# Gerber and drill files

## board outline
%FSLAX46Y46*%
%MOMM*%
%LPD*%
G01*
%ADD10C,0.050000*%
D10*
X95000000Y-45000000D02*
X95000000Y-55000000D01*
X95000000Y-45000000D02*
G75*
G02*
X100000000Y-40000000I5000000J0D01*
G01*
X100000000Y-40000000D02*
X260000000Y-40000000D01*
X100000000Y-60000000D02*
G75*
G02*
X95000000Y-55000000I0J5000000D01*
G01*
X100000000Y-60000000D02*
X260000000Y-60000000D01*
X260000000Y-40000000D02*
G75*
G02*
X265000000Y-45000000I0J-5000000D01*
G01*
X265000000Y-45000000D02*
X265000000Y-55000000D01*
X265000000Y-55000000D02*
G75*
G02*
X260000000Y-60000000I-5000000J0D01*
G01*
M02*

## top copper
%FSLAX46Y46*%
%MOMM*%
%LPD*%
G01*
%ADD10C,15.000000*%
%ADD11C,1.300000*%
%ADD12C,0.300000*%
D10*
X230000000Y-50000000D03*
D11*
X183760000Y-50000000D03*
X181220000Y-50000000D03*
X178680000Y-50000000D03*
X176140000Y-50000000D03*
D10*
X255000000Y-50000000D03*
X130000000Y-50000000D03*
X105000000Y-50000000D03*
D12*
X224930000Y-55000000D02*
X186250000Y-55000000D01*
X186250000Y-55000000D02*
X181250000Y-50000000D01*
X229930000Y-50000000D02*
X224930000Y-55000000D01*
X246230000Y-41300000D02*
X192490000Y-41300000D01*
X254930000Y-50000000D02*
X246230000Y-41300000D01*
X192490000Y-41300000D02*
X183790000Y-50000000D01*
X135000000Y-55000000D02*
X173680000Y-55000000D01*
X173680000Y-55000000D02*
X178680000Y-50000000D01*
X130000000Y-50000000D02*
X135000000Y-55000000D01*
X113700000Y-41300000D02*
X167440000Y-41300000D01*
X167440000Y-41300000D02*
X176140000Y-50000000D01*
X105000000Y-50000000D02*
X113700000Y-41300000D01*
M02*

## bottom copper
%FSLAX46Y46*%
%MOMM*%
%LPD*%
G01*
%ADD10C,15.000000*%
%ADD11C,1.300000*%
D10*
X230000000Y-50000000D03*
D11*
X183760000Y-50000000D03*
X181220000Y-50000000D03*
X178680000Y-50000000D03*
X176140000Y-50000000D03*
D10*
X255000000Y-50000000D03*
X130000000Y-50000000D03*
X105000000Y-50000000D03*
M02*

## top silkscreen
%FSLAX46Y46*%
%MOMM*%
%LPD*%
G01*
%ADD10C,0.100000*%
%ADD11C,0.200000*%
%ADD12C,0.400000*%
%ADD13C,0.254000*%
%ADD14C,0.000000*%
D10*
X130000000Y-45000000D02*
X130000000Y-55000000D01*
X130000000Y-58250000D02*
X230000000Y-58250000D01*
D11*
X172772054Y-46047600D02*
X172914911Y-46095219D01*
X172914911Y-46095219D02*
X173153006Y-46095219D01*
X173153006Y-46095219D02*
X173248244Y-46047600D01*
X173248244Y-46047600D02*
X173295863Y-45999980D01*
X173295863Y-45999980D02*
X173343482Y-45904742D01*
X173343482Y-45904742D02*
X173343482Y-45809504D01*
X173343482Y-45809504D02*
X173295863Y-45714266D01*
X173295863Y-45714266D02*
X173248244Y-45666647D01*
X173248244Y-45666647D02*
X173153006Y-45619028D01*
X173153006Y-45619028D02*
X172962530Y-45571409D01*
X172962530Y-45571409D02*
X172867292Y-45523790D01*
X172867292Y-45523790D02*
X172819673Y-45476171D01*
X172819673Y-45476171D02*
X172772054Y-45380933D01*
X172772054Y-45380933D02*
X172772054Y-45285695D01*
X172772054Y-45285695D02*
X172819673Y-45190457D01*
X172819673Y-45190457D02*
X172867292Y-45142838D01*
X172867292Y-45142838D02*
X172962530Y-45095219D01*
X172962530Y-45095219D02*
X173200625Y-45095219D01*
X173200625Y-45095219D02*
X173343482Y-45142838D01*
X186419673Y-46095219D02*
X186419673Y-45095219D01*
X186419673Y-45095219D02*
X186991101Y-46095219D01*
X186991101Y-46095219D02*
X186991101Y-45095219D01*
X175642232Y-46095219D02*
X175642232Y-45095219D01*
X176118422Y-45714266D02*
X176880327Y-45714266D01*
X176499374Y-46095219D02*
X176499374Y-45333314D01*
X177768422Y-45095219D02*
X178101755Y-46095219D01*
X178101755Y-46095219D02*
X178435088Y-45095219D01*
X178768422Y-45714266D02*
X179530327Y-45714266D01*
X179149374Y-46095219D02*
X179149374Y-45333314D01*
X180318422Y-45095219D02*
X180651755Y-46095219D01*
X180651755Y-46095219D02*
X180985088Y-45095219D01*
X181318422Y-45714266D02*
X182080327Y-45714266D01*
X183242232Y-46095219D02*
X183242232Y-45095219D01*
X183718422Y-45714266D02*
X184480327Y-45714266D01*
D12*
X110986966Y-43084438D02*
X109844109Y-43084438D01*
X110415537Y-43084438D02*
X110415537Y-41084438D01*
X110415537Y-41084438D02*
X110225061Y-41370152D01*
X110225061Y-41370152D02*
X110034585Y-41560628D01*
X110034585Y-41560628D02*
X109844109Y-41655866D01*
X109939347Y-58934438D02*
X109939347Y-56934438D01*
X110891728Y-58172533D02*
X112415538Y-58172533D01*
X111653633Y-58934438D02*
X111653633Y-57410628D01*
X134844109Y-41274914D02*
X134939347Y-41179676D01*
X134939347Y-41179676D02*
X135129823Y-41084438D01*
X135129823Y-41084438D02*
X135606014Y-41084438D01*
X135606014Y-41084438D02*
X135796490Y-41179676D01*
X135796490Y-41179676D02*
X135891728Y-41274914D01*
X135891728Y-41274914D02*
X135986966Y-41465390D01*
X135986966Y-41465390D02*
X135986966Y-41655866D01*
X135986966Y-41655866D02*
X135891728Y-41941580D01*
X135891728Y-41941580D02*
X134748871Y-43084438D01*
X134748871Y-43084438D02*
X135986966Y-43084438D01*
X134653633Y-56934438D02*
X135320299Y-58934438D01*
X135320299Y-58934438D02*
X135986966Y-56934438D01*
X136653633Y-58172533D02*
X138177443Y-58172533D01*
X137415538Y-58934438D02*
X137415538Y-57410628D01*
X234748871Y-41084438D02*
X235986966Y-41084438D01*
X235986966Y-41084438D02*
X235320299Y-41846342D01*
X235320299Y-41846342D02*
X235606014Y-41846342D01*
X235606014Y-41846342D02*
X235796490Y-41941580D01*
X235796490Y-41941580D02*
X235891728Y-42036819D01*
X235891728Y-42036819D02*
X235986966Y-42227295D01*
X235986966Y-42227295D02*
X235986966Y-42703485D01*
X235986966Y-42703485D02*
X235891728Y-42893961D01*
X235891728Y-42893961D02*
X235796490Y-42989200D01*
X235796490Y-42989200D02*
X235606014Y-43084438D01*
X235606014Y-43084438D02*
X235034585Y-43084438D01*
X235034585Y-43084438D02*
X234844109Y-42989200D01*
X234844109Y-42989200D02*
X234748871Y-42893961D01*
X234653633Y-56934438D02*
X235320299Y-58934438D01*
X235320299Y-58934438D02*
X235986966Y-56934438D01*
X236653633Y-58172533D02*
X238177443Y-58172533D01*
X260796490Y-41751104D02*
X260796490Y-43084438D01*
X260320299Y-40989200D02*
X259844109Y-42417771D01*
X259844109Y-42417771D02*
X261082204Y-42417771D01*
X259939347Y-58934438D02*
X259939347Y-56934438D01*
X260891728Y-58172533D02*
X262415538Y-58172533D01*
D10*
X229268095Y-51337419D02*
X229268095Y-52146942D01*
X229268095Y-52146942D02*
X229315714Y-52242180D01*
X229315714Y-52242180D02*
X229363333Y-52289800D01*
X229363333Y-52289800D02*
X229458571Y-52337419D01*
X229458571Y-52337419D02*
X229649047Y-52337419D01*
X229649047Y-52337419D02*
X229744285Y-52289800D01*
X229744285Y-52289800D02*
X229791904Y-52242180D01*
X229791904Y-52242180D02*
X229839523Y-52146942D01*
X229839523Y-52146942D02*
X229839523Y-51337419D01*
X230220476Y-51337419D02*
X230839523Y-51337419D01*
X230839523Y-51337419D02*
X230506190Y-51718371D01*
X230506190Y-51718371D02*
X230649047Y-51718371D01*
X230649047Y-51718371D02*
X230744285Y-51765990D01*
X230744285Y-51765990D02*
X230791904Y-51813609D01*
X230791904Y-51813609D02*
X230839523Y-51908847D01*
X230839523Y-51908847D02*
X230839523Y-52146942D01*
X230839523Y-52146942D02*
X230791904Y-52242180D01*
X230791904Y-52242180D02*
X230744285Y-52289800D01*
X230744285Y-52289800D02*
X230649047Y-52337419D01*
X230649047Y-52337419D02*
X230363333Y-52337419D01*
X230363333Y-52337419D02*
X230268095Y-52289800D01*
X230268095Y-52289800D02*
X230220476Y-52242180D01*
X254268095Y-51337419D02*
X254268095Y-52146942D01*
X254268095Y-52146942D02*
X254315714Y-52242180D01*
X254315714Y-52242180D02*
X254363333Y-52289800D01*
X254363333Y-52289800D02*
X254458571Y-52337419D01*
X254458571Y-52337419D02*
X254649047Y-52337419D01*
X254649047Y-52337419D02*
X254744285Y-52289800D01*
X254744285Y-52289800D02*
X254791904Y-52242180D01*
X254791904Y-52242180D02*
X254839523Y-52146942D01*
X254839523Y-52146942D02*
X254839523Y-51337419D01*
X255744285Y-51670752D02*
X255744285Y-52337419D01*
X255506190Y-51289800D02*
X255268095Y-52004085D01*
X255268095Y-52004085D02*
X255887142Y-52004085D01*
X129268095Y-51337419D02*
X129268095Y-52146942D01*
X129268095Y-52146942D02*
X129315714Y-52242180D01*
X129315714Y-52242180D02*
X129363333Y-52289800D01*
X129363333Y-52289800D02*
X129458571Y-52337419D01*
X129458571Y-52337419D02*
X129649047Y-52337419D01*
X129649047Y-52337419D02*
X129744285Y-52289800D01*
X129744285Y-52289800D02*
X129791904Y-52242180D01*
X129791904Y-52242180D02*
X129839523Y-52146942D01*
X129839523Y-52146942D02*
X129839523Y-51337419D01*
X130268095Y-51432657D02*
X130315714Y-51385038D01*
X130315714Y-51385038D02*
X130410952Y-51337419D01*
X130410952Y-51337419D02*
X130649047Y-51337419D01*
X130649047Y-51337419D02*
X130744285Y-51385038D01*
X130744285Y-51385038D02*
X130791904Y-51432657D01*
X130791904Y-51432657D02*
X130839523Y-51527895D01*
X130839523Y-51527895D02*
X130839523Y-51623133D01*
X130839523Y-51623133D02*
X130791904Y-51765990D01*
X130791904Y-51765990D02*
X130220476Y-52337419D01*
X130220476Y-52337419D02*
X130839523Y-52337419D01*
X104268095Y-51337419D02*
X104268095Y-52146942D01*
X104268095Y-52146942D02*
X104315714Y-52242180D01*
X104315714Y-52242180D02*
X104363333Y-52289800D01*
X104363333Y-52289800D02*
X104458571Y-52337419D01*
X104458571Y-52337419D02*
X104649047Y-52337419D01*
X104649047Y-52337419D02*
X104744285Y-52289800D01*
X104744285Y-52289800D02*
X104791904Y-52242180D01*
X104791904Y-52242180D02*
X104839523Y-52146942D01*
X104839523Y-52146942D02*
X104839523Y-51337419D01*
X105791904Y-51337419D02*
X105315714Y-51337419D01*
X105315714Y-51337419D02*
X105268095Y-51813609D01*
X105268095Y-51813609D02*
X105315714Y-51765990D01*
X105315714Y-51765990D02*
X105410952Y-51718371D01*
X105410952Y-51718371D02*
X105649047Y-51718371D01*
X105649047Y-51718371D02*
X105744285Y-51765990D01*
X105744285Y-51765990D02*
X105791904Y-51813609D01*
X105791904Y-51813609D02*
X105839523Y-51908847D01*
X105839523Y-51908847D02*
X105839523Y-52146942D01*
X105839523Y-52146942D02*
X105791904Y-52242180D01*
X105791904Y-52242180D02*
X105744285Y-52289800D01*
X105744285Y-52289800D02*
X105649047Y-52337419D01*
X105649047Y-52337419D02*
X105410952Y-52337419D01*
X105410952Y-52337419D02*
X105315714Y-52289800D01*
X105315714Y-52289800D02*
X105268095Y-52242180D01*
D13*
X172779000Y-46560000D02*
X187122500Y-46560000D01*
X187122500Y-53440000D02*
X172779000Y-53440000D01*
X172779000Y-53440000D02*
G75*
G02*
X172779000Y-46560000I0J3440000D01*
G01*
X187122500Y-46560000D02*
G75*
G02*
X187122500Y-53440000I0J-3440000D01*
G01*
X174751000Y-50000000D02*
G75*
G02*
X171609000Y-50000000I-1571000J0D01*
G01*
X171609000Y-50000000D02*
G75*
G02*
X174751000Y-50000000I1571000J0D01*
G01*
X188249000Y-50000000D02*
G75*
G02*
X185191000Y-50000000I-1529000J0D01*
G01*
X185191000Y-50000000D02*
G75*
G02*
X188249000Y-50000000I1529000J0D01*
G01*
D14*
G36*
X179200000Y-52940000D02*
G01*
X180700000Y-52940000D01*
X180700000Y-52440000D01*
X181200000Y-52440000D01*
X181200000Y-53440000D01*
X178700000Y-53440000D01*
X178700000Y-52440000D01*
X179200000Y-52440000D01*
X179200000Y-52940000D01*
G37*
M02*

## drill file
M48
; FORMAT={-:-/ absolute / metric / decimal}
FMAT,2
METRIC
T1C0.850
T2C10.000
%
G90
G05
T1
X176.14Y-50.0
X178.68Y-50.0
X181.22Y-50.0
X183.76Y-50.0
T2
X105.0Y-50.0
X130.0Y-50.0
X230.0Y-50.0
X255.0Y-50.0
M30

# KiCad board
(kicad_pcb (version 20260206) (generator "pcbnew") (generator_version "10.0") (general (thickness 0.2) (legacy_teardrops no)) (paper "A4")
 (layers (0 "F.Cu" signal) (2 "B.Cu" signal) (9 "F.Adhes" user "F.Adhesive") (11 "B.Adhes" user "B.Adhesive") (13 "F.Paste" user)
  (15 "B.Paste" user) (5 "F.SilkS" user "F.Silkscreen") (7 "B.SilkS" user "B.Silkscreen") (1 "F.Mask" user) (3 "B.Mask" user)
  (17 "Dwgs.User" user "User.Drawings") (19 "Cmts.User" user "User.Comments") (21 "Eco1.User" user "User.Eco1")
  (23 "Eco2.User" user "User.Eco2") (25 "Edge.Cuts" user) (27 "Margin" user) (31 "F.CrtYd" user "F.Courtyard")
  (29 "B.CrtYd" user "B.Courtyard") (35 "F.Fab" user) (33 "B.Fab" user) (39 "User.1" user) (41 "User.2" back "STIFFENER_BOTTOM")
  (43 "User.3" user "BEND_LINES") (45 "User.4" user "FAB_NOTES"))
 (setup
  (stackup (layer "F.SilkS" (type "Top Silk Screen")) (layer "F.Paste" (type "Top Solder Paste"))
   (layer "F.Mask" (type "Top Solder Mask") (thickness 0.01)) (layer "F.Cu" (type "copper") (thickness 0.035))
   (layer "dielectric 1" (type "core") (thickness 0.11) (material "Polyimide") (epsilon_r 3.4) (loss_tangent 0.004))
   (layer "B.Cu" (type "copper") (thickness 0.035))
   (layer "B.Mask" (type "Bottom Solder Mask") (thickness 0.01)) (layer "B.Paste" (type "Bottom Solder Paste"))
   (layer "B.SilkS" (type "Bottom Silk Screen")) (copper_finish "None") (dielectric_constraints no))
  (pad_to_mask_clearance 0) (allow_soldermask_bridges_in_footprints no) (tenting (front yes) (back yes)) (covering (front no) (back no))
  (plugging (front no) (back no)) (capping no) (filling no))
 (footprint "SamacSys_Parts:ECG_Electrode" (layer "F.Cu") (at 230.03 52.38)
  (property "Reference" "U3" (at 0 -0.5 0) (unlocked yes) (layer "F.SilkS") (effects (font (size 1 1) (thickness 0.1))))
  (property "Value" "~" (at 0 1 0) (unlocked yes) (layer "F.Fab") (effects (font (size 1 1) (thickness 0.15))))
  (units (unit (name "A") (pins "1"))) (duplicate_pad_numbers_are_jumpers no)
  (pad "1" thru_hole circle (at -0.03 -2.38) (size 15 15) (drill 10) (layers "*.Cu" "*.Mask") (remove_unused_layers no) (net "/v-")))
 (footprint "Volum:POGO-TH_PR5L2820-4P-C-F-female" (layer "F.Cu") (at 179.95 50 180)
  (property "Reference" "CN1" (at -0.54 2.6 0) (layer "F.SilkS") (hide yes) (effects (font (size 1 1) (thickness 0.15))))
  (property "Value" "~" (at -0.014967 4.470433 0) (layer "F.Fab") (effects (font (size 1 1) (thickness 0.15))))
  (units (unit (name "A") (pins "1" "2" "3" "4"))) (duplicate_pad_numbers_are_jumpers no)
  (fp_line (start 7.171 3.44) (end -7.1725 3.44) (stroke (width 0.254) (type default)) (layer "F.SilkS"))
  (fp_line (start -7.1725 -3.44) (end 7.171 -3.44) (stroke (width 0.254) (type default)) (layer "F.SilkS"))
  (fp_arc (start 7.171 -3.44) (mid 10.611 0) (end 7.171 3.44) (stroke (width 0.254) (type default)) (layer "F.SilkS"))
  (fp_arc (start -7.1725 3.44) (mid -10.6125 0) (end -7.1725 -3.44) (stroke (width 0.254) (type default)) (layer "F.SilkS"))
  (fp_circle (center 6.77 0) (end 8.341 0) (stroke (width 0.254) (type default)) (fill no) (layer "F.SilkS"))
  (fp_circle (center -6.77 0) (end -5.241 0) (stroke (width 0.254) (type default)) (fill no) (layer "F.SilkS"))
  (fp_poly
   (pts (xy 1.25 -2.44) (xy 1.25 -3.44) (xy -1.25 -3.44) (xy -1.25 -2.44) (xy -0.75 -2.44) (xy -0.75 -2.94) (xy 0.75 -2.94) (xy 0.75 -2.44))
   (stroke (width 0) (type default)) (fill yes) (layer "F.SilkS"))
  (pad "1" thru_hole circle (at -3.81 0 180) (size 1.3 1.3) (drill 0.85) (layers "*.Cu" "*.Mask") (remove_unused_layers no) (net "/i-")
   (thermal_bridge_angle 90))
  (pad "2" thru_hole circle (at -1.27 0 180) (size 1.3 1.3) (drill 0.85) (layers "*.Cu" "*.Mask") (remove_unused_layers no) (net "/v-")
   (thermal_bridge_angle 90))
  (pad "3" thru_hole circle (at 1.27 0 180) (size 1.3 1.3) (drill 0.85) (layers "*.Cu" "*.Mask") (remove_unused_layers no) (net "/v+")
   (thermal_bridge_angle 90))
  (pad "4" thru_hole circle (at 3.81 0 180) (size 1.3 1.3) (drill 0.85) (layers "*.Cu" "*.Mask") (remove_unused_layers no) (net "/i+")
   (thermal_bridge_angle 90)))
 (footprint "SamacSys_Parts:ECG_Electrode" (layer "F.Cu") (at 255.03 52.38)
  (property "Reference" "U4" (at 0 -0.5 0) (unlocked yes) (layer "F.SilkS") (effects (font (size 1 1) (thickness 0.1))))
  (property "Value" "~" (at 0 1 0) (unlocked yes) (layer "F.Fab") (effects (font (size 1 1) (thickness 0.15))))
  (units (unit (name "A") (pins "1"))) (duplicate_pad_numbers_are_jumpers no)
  (pad "1" thru_hole circle (at -0.03 -2.38) (size 15 15) (drill 10) (layers "*.Cu" "*.Mask") (remove_unused_layers no) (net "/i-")))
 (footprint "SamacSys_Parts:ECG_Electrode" (layer "F.Cu") (at 130.03 52.38)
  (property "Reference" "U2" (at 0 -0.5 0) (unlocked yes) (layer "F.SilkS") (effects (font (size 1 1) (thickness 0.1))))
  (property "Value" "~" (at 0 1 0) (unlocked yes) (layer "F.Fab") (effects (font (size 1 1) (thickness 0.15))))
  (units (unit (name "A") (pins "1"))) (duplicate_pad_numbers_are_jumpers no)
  (pad "1" thru_hole circle (at -0.03 -2.38) (size 15 15) (drill 10) (layers "*.Cu" "*.Mask") (remove_unused_layers no) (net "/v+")))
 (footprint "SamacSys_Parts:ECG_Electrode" (layer "F.Cu") (at 105.03 52.38)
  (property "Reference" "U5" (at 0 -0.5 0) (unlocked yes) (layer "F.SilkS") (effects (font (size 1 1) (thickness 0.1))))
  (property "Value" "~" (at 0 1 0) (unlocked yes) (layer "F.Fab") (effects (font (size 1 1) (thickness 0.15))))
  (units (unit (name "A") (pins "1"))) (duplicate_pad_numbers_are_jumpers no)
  (pad "1" thru_hole circle (at -0.03 -2.38) (size 15 15) (drill 10) (layers "*.Cu" "*.Mask") (remove_unused_layers no) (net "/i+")))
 (gr_line (start 130 45) (end 130 55) (stroke (width 0.1) (type default)) (layer "F.SilkS"))
 (gr_line (start 130 58.25) (end 230 58.25) (stroke (width 0.1) (type default)) (layer "F.SilkS"))
 (gr_line (start 95 45) (end 95 55) (stroke (width 0.05) (type default)) (layer "Edge.Cuts"))
 (gr_arc (start 95 45) (mid 96.464466 41.464466) (end 100 40) (stroke (width 0.05) (type default)) (layer "Edge.Cuts"))
 (gr_line (start 100 40) (end 260 40) (stroke (width 0.05) (type default)) (layer "Edge.Cuts"))
 (gr_arc (start 100 60) (mid 96.464466 58.535534) (end 95 55) (stroke (width 0.05) (type default)) (layer "Edge.Cuts"))
 (gr_line (start 100 60) (end 260 60) (stroke (width 0.05) (type default)) (layer "Edge.Cuts"))
 (gr_arc (start 260 40) (mid 263.535534 41.464466) (end 265 45) (stroke (width 0.05) (type default)) (layer "Edge.Cuts"))
 (gr_line (start 265 45) (end 265 55) (stroke (width 0.05) (type default)) (layer "Edge.Cuts"))
 (gr_arc (start 265 55) (mid 263.535534 58.535534) (end 260 60) (stroke (width 0.05) (type default)) (layer "Edge.Cuts"))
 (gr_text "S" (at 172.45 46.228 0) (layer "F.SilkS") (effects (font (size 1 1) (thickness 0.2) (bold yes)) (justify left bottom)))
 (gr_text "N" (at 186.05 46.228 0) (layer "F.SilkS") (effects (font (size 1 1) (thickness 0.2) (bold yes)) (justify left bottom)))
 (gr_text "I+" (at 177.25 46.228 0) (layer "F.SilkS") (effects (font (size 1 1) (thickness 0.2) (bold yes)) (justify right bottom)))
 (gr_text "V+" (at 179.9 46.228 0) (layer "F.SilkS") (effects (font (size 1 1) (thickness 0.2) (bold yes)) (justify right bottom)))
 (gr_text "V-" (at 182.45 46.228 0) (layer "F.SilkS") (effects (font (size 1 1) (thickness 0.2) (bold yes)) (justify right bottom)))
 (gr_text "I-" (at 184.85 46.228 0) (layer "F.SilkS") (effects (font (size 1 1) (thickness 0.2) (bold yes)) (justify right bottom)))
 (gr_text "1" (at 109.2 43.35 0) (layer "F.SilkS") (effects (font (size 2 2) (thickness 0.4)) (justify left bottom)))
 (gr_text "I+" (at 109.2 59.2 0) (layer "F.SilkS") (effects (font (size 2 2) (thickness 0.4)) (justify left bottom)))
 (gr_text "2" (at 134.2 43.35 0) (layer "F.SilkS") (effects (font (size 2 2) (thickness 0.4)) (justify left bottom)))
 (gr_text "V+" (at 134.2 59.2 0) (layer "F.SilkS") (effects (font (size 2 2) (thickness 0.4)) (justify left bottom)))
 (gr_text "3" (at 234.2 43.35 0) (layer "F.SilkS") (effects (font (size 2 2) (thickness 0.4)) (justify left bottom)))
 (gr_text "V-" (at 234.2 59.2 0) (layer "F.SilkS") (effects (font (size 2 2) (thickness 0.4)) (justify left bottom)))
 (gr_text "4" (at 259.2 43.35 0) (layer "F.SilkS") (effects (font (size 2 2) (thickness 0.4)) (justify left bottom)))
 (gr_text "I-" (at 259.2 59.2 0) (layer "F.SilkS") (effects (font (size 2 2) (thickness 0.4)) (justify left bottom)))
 (segment (start 224.93 55) (end 186.25 55) (width 0.3) (layer "F.Cu") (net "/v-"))
 (segment (start 186.25 55) (end 181.25 50) (width 0.3) (layer "F.Cu") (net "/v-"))
 (segment (start 229.93 50) (end 224.93 55) (width 0.3) (layer "F.Cu") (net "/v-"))
 (segment (start 246.23 41.3) (end 192.49 41.3) (width 0.3) (layer "F.Cu") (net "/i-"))
 (segment (start 254.93 50) (end 246.23 41.3) (width 0.3) (layer "F.Cu") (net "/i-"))
 (segment (start 192.49 41.3) (end 183.79 50) (width 0.3) (layer "F.Cu") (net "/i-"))
 (segment (start 135 55) (end 173.68 55) (width 0.3) (layer "F.Cu") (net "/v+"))
 (segment (start 173.68 55) (end 178.68 50) (width 0.3) (layer "F.Cu") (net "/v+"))
 (segment (start 130 50) (end 135 55) (width 0.3) (layer "F.Cu") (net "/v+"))
 (segment (start 113.7 41.3) (end 167.44 41.3) (width 0.3) (layer "F.Cu") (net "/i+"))
 (segment (start 167.44 41.3) (end 176.14 50) (width 0.3) (layer "F.Cu") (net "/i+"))
 (segment (start 105 50) (end 113.7 41.3) (width 0.3) (layer "F.Cu") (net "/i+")))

